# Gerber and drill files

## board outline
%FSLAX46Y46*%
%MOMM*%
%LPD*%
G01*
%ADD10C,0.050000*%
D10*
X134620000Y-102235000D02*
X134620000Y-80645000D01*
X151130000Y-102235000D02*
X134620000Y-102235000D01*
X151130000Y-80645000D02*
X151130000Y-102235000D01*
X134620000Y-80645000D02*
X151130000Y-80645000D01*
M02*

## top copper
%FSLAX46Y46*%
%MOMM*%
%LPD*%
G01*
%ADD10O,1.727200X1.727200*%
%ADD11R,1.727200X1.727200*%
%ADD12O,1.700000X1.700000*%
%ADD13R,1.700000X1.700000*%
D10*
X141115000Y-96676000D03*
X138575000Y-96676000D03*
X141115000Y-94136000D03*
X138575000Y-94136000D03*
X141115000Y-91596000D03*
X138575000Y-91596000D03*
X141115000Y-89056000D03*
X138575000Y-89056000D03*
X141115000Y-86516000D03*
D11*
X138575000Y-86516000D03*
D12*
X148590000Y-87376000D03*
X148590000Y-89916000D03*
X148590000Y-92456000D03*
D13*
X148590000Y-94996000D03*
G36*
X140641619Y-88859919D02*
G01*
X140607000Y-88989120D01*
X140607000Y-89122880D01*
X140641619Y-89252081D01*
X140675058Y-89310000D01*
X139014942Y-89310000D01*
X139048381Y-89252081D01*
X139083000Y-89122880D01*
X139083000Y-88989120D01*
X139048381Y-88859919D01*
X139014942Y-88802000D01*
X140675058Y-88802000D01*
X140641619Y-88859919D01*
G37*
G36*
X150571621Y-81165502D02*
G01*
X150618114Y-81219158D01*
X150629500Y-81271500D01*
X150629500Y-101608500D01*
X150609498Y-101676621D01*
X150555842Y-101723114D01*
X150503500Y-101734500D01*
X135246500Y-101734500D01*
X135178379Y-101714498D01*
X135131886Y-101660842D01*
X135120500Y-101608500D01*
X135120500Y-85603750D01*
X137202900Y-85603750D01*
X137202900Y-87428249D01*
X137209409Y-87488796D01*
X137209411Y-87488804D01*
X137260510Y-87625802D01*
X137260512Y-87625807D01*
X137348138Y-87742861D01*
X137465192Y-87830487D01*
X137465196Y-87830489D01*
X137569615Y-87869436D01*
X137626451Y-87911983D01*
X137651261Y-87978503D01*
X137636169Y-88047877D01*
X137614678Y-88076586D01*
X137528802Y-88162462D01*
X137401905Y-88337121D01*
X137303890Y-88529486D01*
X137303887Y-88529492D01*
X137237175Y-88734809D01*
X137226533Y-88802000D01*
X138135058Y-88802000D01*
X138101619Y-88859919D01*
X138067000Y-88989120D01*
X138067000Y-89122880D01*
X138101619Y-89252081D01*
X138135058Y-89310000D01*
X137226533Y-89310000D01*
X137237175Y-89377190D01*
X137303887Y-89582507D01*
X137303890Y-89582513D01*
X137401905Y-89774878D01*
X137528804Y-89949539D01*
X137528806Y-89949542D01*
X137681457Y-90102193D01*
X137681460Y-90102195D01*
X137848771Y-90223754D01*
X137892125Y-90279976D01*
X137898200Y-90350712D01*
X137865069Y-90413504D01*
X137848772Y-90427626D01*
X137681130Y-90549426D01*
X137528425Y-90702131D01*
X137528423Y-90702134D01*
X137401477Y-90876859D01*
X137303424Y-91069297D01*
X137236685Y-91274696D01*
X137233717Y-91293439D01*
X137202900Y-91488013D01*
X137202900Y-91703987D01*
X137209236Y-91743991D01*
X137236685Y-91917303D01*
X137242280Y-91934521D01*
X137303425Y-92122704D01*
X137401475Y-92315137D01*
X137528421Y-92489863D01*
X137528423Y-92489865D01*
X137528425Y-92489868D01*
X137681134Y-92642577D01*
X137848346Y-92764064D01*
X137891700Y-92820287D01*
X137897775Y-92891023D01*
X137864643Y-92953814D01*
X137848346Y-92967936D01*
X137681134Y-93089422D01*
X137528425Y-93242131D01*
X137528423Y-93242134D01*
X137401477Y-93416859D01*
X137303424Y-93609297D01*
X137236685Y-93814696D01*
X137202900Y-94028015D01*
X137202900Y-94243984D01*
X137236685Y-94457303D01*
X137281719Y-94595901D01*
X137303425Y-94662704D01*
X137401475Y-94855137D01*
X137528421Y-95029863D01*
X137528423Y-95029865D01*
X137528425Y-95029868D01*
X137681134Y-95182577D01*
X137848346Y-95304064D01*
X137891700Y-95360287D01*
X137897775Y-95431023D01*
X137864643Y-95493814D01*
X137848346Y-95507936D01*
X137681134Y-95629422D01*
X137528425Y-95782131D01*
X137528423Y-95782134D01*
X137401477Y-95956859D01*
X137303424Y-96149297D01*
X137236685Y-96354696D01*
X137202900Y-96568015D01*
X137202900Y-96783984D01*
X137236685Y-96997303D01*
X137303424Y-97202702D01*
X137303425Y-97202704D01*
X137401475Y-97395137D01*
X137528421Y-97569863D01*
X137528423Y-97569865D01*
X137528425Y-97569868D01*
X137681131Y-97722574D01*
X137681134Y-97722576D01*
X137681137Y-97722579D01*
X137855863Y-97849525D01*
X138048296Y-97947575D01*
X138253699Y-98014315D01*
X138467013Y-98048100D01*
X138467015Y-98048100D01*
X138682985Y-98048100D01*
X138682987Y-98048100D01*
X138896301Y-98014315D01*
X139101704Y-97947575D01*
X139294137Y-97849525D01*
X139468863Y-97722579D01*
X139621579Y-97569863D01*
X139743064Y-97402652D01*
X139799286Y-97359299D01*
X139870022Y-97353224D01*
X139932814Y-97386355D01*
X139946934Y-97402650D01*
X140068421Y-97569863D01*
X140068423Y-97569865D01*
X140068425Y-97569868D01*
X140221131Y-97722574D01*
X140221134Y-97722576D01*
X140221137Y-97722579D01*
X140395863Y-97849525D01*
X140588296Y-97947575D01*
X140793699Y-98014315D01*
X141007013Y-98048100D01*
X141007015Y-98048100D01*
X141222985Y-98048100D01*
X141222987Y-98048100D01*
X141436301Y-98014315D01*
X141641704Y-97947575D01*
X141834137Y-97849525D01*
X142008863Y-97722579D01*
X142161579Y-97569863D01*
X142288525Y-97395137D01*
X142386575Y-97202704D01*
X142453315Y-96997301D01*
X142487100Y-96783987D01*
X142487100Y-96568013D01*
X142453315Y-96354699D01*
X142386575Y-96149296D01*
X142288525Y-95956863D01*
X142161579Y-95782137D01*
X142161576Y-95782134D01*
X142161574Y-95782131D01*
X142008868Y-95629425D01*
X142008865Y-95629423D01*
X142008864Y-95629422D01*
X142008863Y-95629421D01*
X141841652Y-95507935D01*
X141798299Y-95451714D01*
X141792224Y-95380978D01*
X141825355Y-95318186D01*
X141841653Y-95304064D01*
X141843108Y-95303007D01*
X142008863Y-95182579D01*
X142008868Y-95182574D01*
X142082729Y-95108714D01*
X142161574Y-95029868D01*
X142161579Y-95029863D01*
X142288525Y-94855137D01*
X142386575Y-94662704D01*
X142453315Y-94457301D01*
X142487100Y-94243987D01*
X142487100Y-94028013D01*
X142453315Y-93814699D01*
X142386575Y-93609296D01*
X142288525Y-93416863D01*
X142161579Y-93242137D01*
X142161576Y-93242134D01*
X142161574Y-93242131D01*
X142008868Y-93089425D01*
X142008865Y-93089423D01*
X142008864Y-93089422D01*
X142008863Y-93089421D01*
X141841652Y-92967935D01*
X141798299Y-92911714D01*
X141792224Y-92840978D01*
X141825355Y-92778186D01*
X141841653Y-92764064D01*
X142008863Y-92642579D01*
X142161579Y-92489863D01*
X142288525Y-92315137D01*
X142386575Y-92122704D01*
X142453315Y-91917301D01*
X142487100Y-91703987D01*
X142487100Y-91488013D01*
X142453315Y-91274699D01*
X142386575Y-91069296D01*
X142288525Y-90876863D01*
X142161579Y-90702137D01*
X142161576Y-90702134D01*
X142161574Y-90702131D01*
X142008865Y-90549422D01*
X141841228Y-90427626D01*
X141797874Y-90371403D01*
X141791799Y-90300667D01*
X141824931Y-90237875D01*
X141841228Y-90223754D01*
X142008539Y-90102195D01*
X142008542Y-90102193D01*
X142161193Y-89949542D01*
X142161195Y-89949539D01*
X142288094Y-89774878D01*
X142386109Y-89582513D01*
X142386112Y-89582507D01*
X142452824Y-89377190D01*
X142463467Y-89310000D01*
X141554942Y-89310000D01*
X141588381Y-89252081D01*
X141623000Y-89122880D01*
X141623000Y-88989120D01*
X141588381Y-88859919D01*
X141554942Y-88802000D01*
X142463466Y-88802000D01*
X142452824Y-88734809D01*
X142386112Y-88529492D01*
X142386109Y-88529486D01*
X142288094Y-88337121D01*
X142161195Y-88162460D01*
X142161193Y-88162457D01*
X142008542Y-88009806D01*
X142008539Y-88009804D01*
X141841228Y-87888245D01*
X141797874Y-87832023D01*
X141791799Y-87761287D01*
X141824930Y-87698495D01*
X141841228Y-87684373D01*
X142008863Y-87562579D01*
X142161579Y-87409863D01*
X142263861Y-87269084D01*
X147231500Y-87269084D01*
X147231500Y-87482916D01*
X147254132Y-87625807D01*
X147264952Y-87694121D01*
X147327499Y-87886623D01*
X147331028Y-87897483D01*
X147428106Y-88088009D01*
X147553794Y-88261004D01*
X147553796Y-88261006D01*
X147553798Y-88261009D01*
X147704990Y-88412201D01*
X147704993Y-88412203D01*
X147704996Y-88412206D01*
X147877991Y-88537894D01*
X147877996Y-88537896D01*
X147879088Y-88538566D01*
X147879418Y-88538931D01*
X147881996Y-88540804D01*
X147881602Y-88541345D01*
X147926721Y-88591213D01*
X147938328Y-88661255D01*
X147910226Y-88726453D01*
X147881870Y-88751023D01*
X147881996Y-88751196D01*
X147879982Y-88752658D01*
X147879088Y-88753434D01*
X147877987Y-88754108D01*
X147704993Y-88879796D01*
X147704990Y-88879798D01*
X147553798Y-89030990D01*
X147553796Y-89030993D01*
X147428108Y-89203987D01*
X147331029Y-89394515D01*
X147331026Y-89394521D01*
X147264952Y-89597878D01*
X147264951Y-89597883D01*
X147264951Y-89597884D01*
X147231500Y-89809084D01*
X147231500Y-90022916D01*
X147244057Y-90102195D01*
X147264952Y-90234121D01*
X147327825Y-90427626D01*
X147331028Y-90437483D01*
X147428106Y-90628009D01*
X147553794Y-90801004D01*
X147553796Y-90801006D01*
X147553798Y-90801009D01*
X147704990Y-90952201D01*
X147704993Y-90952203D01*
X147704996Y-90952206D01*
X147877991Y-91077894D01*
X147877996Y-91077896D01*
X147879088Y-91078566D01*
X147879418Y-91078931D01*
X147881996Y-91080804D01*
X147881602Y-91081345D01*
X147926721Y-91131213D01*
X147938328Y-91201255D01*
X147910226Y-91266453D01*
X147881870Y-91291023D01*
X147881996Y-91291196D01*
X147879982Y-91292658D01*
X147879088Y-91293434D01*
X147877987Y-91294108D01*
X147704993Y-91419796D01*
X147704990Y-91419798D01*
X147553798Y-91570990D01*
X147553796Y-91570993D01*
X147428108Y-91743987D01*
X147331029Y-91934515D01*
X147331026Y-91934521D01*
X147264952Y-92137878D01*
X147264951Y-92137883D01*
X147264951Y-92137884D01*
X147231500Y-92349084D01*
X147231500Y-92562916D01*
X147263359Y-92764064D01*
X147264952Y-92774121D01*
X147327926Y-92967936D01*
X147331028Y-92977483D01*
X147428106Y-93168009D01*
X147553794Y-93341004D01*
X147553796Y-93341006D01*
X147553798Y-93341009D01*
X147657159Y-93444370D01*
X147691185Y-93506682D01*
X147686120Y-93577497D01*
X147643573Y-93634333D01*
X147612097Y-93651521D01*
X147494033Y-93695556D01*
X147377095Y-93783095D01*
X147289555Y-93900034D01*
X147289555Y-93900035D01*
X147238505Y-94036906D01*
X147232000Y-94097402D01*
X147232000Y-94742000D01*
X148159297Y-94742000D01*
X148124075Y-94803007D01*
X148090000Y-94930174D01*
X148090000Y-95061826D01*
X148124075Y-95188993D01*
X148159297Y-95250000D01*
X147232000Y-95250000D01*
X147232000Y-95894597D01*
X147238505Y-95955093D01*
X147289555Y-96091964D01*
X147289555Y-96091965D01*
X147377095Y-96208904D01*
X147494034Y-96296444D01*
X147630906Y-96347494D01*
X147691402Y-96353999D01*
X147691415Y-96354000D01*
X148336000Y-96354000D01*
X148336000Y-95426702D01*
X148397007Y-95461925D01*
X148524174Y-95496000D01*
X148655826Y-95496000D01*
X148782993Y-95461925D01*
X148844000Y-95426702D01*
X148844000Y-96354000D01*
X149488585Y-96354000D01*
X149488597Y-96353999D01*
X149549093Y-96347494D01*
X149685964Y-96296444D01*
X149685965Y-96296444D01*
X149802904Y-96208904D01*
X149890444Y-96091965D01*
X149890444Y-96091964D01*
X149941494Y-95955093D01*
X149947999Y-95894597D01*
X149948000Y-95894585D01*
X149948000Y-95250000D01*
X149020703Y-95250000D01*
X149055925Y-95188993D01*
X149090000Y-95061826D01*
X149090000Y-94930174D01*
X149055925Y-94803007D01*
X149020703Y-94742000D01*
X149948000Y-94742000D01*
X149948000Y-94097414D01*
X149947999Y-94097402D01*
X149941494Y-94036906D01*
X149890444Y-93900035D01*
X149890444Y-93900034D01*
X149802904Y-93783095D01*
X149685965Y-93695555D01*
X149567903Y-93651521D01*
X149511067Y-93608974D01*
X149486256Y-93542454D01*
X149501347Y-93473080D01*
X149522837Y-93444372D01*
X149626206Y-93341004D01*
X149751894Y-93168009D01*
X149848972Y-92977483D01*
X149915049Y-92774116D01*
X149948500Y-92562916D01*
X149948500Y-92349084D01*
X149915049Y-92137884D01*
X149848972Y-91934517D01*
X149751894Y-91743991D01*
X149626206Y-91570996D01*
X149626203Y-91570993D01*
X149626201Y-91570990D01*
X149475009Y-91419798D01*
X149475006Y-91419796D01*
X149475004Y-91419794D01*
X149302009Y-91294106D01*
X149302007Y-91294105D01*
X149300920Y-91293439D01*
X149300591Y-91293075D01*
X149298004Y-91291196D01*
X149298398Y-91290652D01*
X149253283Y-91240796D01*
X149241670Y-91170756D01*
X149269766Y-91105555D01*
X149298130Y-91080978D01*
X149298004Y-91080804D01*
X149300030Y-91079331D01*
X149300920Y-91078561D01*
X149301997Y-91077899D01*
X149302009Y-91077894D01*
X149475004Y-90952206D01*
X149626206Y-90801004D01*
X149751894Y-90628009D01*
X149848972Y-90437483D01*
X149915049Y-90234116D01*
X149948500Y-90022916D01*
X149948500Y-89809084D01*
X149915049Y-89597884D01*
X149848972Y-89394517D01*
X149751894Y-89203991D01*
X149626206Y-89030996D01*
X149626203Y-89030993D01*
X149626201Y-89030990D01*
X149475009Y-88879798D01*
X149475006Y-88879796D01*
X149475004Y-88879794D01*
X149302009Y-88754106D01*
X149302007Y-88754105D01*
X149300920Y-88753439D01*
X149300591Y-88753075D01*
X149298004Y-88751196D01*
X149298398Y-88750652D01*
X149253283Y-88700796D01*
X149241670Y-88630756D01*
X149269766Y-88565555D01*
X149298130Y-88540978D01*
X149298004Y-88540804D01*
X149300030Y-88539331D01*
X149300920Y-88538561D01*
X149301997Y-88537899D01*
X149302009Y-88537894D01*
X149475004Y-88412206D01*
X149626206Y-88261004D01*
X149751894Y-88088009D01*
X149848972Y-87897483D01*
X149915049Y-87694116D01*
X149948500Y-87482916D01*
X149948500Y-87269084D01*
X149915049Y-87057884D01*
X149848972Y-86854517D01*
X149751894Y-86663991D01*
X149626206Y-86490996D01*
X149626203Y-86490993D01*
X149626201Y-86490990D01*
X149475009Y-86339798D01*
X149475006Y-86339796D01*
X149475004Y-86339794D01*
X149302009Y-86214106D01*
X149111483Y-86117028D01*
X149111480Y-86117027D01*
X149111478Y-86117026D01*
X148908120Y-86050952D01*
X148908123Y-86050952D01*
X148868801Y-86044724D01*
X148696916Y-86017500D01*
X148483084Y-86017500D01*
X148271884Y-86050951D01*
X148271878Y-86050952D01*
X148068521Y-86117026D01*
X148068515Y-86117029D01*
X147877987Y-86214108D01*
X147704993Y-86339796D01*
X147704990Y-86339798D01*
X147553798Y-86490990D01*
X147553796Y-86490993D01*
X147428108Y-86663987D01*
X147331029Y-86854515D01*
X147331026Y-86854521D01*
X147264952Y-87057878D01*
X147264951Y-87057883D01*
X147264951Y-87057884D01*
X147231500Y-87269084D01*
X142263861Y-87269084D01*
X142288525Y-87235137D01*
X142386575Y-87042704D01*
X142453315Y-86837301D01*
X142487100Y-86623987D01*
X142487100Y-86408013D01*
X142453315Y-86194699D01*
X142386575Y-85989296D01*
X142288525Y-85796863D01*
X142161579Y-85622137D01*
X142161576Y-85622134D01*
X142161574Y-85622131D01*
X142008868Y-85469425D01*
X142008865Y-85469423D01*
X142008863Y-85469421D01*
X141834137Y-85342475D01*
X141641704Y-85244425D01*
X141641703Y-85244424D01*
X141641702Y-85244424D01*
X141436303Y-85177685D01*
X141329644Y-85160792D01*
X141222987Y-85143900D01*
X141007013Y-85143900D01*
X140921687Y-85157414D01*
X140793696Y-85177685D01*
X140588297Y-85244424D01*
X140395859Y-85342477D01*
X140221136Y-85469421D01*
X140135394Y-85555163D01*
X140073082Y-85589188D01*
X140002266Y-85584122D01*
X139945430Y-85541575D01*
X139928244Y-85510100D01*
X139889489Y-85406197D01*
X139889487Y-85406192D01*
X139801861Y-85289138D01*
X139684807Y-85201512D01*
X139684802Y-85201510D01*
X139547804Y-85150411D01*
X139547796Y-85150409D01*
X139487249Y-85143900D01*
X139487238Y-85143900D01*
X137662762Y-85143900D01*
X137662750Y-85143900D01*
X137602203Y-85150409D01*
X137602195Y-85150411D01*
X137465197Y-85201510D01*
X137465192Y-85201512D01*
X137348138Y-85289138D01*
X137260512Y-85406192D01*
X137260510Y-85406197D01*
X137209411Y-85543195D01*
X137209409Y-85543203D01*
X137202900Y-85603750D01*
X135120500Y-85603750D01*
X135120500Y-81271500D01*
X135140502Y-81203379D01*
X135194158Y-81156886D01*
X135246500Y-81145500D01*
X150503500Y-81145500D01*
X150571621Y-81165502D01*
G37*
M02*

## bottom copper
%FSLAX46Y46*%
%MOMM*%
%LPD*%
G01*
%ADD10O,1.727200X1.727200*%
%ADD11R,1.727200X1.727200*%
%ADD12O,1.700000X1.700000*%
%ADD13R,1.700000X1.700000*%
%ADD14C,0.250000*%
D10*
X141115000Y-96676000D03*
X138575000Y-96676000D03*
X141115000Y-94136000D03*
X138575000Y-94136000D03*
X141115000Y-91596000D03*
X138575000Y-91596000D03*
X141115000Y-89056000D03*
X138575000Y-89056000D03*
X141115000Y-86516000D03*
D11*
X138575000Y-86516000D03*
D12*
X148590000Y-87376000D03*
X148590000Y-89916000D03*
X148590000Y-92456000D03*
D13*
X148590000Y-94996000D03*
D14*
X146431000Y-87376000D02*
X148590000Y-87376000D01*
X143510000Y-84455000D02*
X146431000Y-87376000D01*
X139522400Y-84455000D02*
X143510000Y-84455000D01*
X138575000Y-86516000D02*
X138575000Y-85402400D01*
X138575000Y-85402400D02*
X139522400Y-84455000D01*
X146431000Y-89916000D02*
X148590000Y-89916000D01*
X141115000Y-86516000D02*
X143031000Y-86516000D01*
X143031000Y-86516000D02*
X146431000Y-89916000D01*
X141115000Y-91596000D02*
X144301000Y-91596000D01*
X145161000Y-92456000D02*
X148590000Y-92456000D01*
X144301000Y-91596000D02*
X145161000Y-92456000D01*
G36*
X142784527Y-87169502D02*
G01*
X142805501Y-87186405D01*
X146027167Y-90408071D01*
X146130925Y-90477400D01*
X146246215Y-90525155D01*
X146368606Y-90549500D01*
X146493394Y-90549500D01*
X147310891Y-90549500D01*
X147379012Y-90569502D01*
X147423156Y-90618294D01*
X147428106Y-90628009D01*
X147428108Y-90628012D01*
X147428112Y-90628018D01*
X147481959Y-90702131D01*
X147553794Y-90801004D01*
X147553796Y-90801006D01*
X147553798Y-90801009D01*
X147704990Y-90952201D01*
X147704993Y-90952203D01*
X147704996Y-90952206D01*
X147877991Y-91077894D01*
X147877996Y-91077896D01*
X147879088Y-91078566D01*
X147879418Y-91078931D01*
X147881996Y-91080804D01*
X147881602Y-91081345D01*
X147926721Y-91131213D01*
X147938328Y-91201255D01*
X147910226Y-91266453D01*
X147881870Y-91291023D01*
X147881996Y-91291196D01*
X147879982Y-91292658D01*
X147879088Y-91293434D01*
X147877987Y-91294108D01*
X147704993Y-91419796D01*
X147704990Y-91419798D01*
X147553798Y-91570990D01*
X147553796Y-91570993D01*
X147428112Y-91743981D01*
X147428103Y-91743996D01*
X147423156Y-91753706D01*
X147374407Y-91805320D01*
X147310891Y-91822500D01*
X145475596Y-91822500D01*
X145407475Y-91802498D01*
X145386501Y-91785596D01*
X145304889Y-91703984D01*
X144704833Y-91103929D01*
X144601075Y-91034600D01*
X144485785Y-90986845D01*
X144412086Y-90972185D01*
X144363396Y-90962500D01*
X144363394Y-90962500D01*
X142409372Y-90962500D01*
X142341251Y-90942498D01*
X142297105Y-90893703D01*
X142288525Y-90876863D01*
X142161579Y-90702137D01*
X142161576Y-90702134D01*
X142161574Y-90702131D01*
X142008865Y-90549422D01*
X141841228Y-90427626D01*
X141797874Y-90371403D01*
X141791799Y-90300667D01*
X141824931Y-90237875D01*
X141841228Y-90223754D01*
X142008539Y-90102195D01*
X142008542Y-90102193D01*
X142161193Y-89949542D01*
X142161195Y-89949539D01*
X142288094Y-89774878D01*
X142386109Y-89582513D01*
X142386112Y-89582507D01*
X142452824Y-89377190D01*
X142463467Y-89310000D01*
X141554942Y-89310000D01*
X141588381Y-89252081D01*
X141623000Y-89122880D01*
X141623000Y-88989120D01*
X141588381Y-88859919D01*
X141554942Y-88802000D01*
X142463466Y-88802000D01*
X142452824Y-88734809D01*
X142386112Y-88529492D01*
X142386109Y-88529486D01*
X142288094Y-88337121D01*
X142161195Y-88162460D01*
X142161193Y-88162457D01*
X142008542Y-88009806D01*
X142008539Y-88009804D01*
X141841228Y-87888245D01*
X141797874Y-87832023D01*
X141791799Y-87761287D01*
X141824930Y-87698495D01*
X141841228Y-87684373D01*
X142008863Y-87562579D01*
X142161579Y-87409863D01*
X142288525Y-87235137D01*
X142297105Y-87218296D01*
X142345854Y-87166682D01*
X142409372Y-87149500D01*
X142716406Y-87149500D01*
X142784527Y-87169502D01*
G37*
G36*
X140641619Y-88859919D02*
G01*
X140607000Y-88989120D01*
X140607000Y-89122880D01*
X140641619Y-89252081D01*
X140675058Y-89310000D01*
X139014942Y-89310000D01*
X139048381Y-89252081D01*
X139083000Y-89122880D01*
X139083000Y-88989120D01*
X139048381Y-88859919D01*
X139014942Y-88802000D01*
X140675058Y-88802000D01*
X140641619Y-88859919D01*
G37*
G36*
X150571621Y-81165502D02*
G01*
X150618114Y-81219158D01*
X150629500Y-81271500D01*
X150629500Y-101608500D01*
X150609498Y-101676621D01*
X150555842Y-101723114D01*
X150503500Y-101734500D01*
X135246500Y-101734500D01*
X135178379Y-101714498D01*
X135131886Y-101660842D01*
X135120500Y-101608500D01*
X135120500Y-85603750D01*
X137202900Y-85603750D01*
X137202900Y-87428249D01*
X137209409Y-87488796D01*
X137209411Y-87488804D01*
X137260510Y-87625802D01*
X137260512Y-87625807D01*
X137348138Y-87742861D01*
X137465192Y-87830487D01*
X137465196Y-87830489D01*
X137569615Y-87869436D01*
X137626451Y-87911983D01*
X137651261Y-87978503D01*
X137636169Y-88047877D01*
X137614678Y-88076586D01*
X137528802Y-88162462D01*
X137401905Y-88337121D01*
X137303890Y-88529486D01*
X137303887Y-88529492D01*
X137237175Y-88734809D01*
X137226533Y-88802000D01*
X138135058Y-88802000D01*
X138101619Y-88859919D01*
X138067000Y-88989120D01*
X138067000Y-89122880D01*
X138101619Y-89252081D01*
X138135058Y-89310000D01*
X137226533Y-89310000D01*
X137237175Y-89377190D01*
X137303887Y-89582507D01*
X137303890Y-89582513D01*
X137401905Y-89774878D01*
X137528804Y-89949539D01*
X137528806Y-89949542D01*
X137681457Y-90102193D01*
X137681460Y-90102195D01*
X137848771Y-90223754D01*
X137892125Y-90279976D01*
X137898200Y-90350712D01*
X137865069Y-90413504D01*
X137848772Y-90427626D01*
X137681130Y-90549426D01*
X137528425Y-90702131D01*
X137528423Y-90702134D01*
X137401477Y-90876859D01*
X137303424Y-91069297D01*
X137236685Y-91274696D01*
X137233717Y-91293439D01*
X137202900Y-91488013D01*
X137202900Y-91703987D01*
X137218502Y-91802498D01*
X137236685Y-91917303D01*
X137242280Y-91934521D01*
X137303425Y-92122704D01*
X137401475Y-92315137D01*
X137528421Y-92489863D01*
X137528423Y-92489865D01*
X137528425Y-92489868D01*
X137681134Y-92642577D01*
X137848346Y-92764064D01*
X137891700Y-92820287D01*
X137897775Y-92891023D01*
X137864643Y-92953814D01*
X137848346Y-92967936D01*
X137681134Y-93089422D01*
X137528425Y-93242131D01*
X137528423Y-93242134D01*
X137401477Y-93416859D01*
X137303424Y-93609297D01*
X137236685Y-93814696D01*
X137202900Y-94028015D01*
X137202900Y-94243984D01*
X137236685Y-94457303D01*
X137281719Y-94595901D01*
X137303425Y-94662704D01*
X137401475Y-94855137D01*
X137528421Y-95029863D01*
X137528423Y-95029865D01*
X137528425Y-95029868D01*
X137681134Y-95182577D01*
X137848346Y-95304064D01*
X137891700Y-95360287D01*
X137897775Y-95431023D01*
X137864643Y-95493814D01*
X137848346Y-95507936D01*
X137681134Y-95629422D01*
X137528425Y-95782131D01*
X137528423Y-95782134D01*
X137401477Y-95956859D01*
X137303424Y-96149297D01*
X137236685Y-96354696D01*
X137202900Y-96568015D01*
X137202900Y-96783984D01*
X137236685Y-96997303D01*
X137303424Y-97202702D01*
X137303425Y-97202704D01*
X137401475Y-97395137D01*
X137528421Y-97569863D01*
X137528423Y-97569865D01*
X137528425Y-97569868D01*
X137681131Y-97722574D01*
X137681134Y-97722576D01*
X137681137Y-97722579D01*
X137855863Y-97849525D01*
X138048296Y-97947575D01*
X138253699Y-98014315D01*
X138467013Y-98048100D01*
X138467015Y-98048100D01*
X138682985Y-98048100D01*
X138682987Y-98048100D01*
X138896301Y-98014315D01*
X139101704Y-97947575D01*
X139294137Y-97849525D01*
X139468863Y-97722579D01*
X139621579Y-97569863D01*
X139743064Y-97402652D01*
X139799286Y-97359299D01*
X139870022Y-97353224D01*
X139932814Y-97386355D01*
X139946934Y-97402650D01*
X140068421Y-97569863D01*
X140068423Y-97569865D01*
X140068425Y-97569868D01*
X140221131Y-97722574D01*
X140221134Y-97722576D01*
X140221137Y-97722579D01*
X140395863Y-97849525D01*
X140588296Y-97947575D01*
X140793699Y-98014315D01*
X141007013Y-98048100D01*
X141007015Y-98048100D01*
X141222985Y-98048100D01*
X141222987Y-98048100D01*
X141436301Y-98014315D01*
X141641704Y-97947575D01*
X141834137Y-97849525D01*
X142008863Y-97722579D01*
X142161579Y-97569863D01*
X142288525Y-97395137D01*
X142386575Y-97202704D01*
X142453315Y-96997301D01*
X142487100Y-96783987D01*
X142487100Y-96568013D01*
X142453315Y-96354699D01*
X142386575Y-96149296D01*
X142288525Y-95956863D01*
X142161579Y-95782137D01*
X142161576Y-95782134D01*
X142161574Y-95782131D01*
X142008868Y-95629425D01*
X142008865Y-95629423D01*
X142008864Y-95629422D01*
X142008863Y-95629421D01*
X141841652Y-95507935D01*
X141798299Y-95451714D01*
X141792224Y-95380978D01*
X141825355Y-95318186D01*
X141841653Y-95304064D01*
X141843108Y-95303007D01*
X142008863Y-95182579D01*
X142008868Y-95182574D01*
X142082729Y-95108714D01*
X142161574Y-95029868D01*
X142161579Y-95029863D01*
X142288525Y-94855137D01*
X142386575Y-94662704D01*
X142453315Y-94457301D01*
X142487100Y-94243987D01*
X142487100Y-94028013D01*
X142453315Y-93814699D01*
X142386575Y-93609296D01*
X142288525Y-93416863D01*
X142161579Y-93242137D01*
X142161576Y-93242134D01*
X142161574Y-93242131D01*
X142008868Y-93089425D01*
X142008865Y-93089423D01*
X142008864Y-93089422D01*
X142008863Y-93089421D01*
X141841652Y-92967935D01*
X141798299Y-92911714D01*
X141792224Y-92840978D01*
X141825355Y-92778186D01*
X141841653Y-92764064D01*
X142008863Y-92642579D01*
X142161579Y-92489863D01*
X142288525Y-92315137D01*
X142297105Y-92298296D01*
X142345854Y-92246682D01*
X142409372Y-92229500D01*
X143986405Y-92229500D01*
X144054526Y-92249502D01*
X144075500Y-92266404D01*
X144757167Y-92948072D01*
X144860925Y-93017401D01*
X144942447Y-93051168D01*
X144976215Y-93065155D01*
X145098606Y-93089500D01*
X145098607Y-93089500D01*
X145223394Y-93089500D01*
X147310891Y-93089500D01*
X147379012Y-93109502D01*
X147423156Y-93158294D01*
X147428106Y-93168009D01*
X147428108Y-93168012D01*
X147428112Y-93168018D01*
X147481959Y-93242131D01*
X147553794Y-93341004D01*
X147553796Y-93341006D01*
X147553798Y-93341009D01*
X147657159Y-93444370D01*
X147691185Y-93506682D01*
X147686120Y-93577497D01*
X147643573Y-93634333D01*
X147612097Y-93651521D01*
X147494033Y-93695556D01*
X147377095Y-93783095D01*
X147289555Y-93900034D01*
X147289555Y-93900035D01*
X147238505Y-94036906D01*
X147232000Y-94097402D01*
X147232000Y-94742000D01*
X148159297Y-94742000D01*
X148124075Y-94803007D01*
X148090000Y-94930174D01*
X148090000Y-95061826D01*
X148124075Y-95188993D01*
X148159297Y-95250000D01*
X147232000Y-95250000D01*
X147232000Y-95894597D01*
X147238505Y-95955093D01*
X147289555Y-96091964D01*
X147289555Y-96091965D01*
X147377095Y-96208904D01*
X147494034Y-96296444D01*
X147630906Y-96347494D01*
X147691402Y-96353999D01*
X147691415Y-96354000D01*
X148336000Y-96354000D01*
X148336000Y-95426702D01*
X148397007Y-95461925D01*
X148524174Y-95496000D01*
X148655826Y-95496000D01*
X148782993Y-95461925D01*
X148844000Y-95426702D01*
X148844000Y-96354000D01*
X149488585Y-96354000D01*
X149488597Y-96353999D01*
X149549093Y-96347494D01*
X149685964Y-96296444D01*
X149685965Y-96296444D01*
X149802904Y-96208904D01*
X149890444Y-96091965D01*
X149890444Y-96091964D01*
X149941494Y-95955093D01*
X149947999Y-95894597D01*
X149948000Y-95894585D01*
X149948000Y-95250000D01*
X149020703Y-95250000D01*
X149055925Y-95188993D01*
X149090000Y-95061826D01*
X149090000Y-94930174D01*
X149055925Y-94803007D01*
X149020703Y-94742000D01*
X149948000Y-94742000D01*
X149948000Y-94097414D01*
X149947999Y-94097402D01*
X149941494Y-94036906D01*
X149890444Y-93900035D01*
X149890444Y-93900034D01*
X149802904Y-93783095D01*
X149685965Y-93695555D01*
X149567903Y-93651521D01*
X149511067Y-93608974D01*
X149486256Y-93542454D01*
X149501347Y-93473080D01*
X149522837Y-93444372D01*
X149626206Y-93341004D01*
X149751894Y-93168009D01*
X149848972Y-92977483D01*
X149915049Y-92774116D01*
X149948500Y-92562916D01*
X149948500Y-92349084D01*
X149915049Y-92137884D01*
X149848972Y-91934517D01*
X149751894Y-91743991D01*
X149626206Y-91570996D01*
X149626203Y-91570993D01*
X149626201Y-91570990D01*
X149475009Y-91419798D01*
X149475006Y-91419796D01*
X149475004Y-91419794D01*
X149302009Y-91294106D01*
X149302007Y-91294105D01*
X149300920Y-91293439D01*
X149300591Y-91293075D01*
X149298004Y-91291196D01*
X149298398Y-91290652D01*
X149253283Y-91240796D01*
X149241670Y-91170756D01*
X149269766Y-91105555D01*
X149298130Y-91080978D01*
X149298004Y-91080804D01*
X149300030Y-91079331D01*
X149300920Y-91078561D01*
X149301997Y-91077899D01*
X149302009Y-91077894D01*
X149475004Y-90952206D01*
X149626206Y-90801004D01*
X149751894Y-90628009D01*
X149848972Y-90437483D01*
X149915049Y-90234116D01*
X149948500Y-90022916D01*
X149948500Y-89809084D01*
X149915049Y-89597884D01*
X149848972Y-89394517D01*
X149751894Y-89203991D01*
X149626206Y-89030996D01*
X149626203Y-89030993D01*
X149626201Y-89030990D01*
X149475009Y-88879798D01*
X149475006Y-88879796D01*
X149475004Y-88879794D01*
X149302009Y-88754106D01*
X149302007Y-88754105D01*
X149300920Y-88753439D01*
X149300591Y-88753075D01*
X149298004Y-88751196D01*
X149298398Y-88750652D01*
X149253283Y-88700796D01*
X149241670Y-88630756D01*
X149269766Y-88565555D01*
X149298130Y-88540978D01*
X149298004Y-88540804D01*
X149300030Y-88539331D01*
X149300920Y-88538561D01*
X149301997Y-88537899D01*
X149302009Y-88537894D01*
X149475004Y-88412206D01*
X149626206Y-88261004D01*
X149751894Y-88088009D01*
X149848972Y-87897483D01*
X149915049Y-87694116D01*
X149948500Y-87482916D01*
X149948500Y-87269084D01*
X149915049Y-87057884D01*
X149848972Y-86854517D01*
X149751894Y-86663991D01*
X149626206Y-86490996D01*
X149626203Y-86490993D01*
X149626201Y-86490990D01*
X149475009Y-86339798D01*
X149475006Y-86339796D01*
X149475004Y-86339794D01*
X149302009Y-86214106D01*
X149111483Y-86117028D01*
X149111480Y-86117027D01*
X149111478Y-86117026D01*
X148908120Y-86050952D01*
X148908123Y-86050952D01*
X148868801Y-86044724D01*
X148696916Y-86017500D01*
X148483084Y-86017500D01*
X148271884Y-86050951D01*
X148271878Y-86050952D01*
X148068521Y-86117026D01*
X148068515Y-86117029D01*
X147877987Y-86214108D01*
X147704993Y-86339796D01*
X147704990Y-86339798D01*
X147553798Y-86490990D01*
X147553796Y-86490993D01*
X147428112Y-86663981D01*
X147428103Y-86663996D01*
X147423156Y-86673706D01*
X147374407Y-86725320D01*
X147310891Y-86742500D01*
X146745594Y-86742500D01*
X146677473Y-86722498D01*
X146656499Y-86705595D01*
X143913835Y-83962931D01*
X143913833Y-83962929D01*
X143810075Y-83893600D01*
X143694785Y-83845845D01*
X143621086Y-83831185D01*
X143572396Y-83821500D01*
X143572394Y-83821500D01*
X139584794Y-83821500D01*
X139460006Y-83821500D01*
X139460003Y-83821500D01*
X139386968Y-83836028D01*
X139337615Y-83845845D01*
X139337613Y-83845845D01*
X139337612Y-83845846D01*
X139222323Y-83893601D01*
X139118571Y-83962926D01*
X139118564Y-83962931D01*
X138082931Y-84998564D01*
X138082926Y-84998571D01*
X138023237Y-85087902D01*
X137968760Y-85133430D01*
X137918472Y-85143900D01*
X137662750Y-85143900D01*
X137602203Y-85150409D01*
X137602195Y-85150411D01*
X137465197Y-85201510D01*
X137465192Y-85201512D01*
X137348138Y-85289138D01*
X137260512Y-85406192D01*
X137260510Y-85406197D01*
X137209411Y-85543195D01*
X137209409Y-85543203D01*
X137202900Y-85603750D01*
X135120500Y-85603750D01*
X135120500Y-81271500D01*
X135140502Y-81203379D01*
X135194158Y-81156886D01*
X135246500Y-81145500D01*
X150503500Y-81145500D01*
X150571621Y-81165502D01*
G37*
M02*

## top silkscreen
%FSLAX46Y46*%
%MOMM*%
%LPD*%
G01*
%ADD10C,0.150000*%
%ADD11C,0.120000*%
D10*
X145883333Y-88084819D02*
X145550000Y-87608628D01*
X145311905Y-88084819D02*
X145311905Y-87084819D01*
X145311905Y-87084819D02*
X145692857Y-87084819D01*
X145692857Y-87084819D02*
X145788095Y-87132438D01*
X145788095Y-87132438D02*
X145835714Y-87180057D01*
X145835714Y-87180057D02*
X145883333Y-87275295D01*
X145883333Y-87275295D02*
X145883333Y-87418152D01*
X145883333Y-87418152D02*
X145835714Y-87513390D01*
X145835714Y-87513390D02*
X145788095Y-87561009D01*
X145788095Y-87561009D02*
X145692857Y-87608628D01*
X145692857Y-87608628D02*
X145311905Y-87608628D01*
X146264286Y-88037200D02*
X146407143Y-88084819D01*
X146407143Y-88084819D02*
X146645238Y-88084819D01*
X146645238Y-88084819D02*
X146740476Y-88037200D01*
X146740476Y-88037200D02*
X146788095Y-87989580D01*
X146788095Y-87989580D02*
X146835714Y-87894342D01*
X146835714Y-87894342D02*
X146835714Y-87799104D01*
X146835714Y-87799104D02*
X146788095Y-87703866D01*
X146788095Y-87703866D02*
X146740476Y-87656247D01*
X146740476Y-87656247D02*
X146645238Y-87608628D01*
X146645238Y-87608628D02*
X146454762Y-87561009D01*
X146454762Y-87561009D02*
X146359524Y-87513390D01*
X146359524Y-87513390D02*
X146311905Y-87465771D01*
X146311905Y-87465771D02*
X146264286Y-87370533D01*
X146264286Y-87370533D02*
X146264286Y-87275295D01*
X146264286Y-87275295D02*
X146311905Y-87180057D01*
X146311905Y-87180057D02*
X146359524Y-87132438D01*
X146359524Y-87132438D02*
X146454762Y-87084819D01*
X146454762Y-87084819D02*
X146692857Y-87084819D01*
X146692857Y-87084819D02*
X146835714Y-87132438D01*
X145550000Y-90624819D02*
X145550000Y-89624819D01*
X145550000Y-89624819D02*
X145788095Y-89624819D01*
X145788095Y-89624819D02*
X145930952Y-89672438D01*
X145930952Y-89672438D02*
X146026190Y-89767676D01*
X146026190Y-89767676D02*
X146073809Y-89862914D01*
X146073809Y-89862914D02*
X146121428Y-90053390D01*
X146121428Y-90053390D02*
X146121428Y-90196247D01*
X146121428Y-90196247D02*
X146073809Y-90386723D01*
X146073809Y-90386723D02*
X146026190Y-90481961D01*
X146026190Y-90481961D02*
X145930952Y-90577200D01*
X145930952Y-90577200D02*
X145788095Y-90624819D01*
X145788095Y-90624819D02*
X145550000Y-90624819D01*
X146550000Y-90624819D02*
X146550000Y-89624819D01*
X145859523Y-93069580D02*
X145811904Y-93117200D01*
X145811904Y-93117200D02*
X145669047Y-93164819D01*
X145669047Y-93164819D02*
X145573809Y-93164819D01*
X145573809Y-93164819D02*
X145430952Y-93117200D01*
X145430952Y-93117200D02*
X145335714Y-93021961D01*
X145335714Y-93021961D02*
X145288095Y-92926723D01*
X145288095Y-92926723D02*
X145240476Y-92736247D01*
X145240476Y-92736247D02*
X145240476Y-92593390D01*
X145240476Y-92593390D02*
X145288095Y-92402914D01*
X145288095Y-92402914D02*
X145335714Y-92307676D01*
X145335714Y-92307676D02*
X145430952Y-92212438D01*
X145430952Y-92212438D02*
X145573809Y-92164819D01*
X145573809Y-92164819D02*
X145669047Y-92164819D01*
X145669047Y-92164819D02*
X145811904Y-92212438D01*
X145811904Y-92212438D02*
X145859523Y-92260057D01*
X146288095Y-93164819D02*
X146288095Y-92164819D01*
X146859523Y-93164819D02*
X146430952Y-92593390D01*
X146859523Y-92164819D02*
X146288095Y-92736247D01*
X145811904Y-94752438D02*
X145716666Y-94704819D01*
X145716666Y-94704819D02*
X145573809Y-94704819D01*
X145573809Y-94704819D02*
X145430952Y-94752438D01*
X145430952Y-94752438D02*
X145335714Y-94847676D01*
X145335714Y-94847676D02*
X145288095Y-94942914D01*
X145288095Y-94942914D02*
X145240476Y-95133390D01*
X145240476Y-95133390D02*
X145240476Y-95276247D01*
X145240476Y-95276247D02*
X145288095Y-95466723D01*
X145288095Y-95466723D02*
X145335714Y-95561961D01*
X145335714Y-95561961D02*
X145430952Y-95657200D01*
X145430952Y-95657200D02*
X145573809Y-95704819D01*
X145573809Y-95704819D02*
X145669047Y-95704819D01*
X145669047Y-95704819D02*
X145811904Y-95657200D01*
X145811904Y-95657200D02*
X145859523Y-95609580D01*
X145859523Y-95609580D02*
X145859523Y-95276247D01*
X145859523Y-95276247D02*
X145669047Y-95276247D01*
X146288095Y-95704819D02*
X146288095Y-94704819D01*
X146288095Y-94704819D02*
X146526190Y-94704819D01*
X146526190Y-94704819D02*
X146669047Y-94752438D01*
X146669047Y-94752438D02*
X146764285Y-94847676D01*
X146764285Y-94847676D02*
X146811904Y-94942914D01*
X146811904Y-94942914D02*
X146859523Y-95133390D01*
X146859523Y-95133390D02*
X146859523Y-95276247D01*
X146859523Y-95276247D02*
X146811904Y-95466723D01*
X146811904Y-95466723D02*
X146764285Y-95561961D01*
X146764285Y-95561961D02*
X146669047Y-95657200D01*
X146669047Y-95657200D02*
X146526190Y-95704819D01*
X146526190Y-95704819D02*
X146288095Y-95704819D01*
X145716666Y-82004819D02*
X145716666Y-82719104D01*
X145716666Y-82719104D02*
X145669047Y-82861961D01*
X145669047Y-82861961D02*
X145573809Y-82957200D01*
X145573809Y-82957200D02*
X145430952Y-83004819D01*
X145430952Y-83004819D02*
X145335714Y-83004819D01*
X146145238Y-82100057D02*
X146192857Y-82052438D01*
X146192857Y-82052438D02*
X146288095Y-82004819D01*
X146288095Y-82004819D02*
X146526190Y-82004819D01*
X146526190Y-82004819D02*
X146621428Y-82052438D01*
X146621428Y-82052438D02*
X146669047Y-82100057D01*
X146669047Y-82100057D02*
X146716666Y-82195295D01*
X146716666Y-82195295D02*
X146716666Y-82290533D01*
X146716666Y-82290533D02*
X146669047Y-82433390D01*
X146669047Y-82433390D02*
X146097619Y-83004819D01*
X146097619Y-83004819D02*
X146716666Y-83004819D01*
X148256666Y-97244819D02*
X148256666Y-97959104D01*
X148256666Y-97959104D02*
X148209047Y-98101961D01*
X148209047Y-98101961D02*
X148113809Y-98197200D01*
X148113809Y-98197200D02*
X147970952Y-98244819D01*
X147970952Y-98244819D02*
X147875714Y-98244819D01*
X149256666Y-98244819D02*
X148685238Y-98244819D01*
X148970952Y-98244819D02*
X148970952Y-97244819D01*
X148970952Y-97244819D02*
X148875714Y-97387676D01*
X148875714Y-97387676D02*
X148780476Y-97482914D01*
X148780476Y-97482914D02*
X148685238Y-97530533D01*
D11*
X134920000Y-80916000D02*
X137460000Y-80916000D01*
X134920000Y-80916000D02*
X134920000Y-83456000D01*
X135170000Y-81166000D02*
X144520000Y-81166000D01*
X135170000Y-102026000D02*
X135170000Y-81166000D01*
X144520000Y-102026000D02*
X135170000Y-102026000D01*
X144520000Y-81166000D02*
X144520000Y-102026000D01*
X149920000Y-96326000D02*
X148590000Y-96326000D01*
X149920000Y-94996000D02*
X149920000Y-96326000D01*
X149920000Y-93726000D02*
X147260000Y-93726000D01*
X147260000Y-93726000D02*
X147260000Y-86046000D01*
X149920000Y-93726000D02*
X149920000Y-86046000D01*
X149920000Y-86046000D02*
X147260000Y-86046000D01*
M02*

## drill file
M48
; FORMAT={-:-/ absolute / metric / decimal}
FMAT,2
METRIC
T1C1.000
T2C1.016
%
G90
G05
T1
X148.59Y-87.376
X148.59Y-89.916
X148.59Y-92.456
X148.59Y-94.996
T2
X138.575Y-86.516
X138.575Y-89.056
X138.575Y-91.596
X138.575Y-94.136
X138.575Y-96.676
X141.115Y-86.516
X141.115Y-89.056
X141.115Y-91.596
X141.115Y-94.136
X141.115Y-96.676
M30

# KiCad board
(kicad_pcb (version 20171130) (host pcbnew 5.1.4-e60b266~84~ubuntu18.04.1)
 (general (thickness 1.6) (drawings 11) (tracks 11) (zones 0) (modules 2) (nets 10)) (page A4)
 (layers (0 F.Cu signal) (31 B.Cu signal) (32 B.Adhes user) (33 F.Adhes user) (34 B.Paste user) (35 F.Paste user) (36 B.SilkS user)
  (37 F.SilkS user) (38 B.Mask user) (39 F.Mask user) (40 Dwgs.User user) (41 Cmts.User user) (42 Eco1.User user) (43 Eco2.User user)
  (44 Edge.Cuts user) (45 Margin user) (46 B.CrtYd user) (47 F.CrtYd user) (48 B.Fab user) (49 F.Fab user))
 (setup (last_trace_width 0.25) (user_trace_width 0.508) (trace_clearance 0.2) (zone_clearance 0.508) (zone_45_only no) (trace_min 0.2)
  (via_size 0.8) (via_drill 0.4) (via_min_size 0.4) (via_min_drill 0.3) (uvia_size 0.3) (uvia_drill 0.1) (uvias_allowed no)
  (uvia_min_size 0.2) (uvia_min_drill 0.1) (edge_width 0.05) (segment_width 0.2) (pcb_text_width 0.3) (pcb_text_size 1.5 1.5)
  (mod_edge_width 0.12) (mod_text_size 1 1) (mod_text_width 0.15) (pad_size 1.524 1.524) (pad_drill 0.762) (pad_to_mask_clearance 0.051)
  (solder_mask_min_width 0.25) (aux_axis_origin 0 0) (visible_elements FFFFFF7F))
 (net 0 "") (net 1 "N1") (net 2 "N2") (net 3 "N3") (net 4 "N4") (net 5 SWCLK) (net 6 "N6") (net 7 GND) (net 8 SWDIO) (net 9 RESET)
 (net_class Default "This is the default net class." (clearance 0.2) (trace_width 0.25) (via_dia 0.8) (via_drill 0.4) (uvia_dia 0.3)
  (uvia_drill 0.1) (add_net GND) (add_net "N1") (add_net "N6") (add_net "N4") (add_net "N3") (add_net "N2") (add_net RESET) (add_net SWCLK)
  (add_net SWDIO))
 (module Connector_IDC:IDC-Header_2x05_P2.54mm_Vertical (layer F.Cu) (at 138.575 86.516)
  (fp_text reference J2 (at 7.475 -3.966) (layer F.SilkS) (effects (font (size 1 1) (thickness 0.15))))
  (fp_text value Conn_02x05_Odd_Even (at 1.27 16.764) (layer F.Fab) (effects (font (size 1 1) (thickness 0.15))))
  (fp_line (start -3.655 -5.6) (end -1.115 -5.6) (layer F.SilkS) (width 0.12))
  (fp_line (start -3.655 -5.6) (end -3.655 -3.06) (layer F.SilkS) (width 0.12))
  (fp_line (start -3.405 -5.35) (end 5.945 -5.35) (layer F.SilkS) (width 0.12))
  (fp_line (start -3.405 15.51) (end -3.405 -5.35) (layer F.SilkS) (width 0.12))
  (fp_line (start 5.945 15.51) (end -3.405 15.51) (layer F.SilkS) (width 0.12))
  (fp_line (start 5.945 -5.35) (end 5.945 15.51) (layer F.SilkS) (width 0.12))
  (pad 10 thru_hole oval (at 2.54 10.16) (size 1.7272 1.7272) (drill 1.016) (layers *.Cu *.Mask) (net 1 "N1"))
  (pad 9 thru_hole oval (at 0 10.16) (size 1.7272 1.7272) (drill 1.016) (layers *.Cu *.Mask) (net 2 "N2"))
  (pad 8 thru_hole oval (at 2.54 7.62) (size 1.7272 1.7272) (drill 1.016) (layers *.Cu *.Mask) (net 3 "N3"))
  (pad 7 thru_hole oval (at 0 7.62) (size 1.7272 1.7272) (drill 1.016) (layers *.Cu *.Mask) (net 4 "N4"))
  (pad 6 thru_hole oval (at 2.54 5.08) (size 1.7272 1.7272) (drill 1.016) (layers *.Cu *.Mask) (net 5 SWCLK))
  (pad 5 thru_hole oval (at 0 5.08) (size 1.7272 1.7272) (drill 1.016) (layers *.Cu *.Mask) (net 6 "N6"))
  (pad 4 thru_hole oval (at 2.54 2.54) (size 1.7272 1.7272) (drill 1.016) (layers *.Cu *.Mask) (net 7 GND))
  (pad 3 thru_hole oval (at 0 2.54) (size 1.7272 1.7272) (drill 1.016) (layers *.Cu *.Mask) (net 7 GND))
  (pad 2 thru_hole oval (at 2.54 0) (size 1.7272 1.7272) (drill 1.016) (layers *.Cu *.Mask) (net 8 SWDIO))
  (pad 1 thru_hole rect (at 0 0) (size 1.7272 1.7272) (drill 1.016) (layers *.Cu *.Mask) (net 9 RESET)))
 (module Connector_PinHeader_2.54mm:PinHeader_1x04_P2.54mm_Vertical (layer F.Cu) (at 148.59 94.996 180)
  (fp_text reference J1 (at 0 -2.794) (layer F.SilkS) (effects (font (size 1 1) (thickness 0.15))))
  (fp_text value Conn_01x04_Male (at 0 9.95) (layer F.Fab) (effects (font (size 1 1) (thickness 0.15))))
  (fp_line (start -1.33 -1.33) (end 0 -1.33) (layer F.SilkS) (width 0.12))
  (fp_line (start -1.33 0) (end -1.33 -1.33) (layer F.SilkS) (width 0.12))
  (fp_line (start -1.33 1.27) (end 1.33 1.27) (layer F.SilkS) (width 0.12))
  (fp_line (start 1.33 1.27) (end 1.33 8.95) (layer F.SilkS) (width 0.12))
  (fp_line (start -1.33 1.27) (end -1.33 8.95) (layer F.SilkS) (width 0.12))
  (fp_line (start -1.33 8.95) (end 1.33 8.95) (layer F.SilkS) (width 0.12))
  (pad 4 thru_hole oval (at 0 7.62 180) (size 1.7 1.7) (drill 1) (layers *.Cu *.Mask) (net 9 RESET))
  (pad 3 thru_hole oval (at 0 5.08 180) (size 1.7 1.7) (drill 1) (layers *.Cu *.Mask) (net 8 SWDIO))
  (pad 2 thru_hole oval (at 0 2.54 180) (size 1.7 1.7) (drill 1) (layers *.Cu *.Mask) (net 5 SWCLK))
  (pad 1 thru_hole rect (at 0 0 180) (size 1.7 1.7) (drill 1) (layers *.Cu *.Mask) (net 7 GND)))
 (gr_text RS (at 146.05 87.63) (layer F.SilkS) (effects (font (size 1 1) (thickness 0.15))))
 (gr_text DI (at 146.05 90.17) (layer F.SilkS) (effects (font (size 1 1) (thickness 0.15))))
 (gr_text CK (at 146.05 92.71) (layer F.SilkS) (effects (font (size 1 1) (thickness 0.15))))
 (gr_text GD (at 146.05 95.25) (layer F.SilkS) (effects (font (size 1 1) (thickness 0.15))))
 (gr_line (start 134.62 102.235) (end 134.62 80.645) (layer Edge.Cuts) (width 0.05))
 (gr_line (start 151.13 102.235) (end 134.62 102.235) (layer Edge.Cuts) (width 0.05))
 (gr_line (start 151.13 80.645) (end 151.13 102.235) (layer Edge.Cuts) (width 0.05))
 (gr_line (start 134.62 80.645) (end 151.13 80.645) (layer Edge.Cuts) (width 0.05))
 (segment (start 146.431 87.376) (end 148.59 87.376) (width 0.25) (layer B.Cu) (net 9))
 (segment (start 143.51 84.455) (end 146.431 87.376) (width 0.25) (layer B.Cu) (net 9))
 (segment (start 139.5224 84.455) (end 143.51 84.455) (width 0.25) (layer B.Cu) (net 9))
 (segment (start 138.575 86.516) (end 138.575 85.4024) (width 0.25) (layer B.Cu) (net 9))
 (segment (start 138.575 85.4024) (end 139.5224 84.455) (width 0.25) (layer B.Cu) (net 9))
 (segment (start 146.431 89.916) (end 148.59 89.916) (width 0.25) (layer B.Cu) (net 8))
 (segment (start 141.115 86.516) (end 143.031 86.516) (width 0.25) (layer B.Cu) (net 8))
 (segment (start 143.031 86.516) (end 146.431 89.916) (width 0.25) (layer B.Cu) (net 8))
 (segment (start 141.115 91.596) (end 144.301 91.596) (width 0.25) (layer B.Cu) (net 5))
 (segment (start 145.161 92.456) (end 148.59 92.456) (width 0.25) (layer B.Cu) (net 5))
 (segment (start 144.301 91.596) (end 145.161 92.456) (width 0.25) (layer B.Cu) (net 5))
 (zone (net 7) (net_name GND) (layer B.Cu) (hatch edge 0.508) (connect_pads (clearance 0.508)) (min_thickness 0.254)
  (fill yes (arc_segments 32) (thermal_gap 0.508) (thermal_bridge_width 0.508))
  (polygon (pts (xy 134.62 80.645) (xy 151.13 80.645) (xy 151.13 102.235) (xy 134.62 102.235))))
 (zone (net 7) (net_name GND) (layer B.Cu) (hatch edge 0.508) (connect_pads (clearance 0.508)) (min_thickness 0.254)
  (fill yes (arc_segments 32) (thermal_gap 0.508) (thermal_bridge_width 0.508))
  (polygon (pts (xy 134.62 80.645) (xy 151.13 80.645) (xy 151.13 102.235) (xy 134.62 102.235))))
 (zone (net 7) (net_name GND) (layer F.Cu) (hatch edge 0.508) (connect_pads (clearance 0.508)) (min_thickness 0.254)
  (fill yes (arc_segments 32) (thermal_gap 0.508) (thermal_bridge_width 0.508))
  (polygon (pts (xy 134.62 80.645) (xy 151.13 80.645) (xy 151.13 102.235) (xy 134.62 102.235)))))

